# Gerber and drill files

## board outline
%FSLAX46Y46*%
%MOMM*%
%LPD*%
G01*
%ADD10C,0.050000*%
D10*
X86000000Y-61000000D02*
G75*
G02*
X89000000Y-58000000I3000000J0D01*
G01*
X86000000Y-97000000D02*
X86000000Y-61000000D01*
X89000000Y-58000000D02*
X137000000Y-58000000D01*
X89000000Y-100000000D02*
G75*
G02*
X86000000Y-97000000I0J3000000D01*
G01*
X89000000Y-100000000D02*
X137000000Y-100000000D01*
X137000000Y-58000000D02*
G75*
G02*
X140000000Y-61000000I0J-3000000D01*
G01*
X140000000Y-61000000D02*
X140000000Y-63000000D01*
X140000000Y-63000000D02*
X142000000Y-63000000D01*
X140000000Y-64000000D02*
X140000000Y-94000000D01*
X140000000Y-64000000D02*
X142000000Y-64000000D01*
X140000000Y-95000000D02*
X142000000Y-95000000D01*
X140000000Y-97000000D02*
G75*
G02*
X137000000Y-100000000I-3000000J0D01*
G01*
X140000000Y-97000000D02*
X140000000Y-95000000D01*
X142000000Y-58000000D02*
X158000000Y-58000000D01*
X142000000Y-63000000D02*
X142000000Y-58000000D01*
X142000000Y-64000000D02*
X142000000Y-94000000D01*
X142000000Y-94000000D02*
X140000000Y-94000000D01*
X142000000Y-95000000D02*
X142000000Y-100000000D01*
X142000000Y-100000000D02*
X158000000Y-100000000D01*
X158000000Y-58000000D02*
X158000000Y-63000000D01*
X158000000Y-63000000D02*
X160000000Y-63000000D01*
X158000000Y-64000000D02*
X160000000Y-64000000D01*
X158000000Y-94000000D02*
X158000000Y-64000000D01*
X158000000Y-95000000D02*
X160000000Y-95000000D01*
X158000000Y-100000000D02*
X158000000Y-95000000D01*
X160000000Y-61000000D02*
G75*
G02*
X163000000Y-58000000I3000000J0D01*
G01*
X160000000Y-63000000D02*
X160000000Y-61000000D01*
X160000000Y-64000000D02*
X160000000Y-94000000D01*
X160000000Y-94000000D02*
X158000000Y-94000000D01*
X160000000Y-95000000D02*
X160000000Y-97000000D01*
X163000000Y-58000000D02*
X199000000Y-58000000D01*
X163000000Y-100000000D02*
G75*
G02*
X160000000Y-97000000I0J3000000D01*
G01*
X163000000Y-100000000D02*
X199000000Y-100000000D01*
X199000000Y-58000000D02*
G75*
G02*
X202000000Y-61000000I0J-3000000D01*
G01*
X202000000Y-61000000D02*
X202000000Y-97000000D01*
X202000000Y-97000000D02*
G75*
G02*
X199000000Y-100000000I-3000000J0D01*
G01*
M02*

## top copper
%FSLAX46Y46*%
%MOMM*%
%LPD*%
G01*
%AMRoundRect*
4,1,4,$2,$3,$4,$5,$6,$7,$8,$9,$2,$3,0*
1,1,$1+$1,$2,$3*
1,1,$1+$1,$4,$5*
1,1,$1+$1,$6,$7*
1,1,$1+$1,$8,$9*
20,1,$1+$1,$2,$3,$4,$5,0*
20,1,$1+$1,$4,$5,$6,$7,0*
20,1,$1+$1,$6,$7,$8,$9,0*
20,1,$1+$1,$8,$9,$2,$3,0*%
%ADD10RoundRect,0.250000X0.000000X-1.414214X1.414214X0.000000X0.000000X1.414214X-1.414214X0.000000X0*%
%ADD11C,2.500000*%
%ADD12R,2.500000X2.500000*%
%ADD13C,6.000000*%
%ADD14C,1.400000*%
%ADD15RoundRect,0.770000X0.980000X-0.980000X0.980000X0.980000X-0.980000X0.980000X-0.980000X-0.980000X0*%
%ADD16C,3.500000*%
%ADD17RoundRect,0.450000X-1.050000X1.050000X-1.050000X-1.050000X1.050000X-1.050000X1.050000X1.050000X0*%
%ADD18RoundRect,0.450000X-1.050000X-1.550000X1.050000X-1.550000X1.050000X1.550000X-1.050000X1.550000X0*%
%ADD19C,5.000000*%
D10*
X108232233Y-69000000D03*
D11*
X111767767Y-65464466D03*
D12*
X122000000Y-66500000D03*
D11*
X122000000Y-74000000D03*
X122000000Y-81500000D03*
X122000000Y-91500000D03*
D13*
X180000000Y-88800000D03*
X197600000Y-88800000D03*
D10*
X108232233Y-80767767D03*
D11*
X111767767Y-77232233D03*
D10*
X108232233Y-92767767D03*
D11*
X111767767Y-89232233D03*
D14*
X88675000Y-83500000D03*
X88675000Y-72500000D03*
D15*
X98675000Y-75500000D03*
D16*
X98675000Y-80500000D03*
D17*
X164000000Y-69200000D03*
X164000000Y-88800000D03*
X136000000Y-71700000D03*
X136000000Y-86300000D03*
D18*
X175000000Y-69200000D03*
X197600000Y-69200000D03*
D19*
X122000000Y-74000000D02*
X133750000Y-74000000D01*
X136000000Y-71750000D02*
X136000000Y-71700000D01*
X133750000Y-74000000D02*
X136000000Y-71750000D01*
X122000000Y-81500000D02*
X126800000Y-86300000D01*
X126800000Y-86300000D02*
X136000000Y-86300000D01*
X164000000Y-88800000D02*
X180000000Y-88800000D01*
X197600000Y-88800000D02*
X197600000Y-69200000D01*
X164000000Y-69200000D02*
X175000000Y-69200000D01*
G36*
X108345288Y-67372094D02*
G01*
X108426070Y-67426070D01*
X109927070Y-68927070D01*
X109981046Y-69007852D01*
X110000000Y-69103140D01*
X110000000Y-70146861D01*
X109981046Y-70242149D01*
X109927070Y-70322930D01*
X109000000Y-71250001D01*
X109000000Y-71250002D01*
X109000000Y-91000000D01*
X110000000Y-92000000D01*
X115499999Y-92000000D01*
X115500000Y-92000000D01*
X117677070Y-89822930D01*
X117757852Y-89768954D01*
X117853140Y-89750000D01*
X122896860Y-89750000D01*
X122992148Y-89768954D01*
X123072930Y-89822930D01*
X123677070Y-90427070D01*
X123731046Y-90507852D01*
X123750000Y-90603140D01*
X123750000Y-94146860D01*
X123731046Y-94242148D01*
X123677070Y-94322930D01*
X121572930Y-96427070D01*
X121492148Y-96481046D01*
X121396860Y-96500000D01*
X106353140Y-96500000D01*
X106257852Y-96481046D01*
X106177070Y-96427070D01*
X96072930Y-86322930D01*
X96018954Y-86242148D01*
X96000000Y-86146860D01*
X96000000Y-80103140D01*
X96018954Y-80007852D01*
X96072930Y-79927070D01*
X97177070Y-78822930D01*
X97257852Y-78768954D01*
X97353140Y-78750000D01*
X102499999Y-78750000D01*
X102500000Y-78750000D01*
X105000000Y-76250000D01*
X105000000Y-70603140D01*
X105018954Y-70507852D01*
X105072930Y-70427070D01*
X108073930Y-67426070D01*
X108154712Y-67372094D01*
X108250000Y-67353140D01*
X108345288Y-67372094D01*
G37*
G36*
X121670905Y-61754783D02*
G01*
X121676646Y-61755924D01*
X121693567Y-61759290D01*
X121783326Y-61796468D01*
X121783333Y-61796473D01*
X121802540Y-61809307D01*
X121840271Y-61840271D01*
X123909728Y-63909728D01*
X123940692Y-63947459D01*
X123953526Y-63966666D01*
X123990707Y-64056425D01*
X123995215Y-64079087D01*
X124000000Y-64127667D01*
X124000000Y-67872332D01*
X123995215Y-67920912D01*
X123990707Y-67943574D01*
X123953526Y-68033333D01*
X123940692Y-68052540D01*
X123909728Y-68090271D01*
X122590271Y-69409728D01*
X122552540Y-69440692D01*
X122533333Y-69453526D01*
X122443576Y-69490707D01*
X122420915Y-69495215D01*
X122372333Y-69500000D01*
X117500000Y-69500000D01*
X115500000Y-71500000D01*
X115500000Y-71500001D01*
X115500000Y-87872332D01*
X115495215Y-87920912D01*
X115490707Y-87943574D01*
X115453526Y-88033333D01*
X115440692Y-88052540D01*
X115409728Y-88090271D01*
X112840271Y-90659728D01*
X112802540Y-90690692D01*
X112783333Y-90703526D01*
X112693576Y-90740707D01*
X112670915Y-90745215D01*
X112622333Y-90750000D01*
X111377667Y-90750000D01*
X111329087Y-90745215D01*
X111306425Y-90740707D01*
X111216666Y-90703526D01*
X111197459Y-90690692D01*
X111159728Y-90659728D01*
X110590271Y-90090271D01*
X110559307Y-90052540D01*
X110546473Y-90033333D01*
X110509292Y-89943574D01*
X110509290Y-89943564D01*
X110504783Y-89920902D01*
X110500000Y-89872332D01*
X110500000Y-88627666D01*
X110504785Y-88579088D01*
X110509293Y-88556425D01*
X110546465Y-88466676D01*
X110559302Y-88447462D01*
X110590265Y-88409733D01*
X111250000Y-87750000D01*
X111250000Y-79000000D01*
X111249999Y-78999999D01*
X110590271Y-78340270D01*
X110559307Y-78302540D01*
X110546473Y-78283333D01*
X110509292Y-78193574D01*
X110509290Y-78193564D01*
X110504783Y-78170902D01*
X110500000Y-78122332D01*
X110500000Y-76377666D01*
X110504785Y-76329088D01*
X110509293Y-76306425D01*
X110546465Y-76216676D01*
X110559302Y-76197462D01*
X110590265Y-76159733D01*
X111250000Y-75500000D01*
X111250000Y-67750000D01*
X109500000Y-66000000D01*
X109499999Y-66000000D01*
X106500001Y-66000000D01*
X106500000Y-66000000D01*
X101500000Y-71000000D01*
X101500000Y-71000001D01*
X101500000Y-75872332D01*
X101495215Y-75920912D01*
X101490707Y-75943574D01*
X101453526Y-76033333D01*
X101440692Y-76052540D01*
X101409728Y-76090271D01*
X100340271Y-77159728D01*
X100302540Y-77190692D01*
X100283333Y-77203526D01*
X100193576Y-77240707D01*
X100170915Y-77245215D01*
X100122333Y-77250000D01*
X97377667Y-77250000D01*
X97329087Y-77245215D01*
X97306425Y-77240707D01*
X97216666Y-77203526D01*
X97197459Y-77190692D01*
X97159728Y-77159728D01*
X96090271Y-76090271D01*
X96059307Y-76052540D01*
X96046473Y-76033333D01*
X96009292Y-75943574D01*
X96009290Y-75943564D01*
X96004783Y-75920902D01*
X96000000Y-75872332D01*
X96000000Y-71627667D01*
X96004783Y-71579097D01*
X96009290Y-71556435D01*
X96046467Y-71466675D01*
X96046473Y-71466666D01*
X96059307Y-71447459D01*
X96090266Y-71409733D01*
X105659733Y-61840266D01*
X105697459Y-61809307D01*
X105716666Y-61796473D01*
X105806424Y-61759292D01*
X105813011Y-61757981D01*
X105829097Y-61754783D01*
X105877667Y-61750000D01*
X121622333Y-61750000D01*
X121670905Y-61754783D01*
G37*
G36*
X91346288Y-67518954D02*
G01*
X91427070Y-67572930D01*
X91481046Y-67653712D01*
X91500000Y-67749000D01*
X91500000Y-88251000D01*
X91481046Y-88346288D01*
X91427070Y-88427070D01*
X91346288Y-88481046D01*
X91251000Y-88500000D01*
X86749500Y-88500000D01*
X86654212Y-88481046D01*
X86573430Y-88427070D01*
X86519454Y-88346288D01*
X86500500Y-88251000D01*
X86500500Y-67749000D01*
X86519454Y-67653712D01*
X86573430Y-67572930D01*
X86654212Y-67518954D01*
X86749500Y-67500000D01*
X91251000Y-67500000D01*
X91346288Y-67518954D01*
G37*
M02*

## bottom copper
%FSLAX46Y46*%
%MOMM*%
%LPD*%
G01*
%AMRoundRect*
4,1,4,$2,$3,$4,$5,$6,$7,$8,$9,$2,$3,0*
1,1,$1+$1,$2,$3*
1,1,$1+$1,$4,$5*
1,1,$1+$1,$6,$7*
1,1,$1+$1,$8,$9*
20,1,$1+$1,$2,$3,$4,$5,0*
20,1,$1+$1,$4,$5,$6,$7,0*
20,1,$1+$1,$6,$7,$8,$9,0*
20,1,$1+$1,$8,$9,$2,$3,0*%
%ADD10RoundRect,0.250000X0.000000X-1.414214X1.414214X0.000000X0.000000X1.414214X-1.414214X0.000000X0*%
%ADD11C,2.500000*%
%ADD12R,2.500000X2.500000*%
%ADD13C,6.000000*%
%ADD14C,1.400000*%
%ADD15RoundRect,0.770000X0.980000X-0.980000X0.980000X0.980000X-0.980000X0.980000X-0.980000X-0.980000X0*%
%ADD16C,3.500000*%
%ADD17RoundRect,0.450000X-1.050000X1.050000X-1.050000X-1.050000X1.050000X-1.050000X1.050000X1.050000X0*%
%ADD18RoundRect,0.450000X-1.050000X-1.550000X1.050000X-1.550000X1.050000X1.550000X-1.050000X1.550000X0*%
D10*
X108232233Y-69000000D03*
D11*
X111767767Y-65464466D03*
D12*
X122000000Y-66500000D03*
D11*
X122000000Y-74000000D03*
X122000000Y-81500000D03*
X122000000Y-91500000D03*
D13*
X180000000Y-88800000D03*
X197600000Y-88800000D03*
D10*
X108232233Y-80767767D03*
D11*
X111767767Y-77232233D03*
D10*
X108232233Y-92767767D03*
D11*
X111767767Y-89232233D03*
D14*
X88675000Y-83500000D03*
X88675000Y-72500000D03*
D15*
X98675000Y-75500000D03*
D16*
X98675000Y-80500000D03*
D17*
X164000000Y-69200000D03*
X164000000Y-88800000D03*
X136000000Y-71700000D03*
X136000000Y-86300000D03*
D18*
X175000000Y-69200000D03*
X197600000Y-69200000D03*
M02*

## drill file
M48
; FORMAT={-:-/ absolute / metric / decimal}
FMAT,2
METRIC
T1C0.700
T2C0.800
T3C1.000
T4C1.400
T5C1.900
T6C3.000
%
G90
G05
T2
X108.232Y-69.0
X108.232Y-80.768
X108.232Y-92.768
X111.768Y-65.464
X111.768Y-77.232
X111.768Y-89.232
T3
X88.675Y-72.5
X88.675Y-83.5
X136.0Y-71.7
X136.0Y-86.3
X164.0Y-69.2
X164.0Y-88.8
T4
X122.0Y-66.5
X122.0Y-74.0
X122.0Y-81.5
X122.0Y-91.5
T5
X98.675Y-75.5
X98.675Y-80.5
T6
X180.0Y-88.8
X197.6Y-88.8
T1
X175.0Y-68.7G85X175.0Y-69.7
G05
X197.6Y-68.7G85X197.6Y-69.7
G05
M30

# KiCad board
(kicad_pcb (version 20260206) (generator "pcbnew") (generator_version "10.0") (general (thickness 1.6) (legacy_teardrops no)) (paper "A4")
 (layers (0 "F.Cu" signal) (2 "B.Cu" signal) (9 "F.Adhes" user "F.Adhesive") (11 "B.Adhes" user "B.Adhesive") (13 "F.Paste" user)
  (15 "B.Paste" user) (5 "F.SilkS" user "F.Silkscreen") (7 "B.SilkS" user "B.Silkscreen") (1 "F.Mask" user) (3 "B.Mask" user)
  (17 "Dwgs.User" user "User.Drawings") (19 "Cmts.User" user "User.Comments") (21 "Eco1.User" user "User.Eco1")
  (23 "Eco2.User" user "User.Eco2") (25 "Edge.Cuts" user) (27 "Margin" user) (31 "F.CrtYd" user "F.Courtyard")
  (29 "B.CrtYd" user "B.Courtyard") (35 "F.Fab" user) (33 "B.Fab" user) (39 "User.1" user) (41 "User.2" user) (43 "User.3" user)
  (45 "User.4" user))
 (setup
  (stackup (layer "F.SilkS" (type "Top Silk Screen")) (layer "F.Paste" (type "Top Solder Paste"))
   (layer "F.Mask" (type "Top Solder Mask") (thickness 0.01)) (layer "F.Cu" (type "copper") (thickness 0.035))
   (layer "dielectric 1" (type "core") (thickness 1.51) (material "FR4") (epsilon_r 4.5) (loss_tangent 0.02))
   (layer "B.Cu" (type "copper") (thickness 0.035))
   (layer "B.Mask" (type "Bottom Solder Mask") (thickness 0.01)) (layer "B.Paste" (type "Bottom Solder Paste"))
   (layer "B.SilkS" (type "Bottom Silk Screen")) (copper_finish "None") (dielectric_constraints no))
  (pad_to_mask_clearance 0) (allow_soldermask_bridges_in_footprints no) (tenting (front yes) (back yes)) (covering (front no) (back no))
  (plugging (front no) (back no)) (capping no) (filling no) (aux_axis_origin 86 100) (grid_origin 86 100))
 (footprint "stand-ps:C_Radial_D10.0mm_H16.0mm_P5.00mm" (layer "F.Cu") (at 108.232233 69 45)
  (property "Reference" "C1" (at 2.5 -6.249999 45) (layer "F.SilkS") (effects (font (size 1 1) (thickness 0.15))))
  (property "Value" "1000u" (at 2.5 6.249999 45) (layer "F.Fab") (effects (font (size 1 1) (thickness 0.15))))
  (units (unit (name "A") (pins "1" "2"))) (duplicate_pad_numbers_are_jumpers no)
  (pad "1" thru_hole roundrect (at 0 0 45) (size 2.5 2.5) (drill 0.8) (layers "*.Cu" "*.Mask") (remove_unused_layers no)
   (roundrect_rratio 0.1) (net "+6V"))
  (pad "2" thru_hole circle (at 5 0 45) (size 2.5 2.5) (drill 0.8) (layers "*.Cu" "*.Mask") (remove_unused_layers no) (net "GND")))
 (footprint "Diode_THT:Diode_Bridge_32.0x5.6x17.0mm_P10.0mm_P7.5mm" (layer "F.Cu") (at 122 66.5 -90)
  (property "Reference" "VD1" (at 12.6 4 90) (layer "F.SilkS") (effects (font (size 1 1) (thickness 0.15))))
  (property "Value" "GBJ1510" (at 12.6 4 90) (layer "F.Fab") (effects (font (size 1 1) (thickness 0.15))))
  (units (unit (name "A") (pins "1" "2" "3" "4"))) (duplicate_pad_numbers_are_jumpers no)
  (pad "1" thru_hole rect (at 0 0 270) (size 2.5 2.5) (drill 1.4) (layers "*.Cu" "*.Mask") (remove_unused_layers no) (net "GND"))
  (pad "2" thru_hole circle (at 7.5 0 270) (size 2.5 2.5) (drill 1.4) (layers "*.Cu" "*.Mask") (remove_unused_layers no) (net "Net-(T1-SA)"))
  (pad "3" thru_hole circle (at 15 0 270) (size 2.5 2.5) (drill 1.4) (layers "*.Cu" "*.Mask") (remove_unused_layers no) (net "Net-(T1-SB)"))
  (pad "4" thru_hole circle (at 25 0 270) (size 2.5 2.5) (drill 1.4) (layers "*.Cu" "*.Mask") (remove_unused_layers no) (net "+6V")))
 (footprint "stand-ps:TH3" (layer "F.Cu") (at 180 88.8)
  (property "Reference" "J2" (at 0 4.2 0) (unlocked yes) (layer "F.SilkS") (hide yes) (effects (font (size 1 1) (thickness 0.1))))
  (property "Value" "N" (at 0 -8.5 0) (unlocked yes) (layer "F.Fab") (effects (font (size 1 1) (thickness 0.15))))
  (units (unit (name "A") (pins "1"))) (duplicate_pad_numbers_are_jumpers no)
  (pad "1" thru_hole circle (at 0 0) (size 6 6) (drill 3) (layers "*.Cu" "*.Mask") (remove_unused_layers no) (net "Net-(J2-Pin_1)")))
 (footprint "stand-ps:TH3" (layer "F.Cu") (at 197.6 88.8)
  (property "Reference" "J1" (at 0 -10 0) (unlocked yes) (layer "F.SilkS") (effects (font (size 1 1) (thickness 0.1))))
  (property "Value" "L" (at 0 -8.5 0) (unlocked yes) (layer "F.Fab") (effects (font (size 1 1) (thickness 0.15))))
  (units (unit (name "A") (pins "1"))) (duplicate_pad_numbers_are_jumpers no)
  (pad "1" thru_hole circle (at 0 0) (size 6 6) (drill 3) (layers "*.Cu" "*.Mask") (remove_unused_layers no) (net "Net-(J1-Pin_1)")))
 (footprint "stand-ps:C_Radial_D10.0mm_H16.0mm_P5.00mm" (layer "F.Cu") (at 108.232233 80.767767 45)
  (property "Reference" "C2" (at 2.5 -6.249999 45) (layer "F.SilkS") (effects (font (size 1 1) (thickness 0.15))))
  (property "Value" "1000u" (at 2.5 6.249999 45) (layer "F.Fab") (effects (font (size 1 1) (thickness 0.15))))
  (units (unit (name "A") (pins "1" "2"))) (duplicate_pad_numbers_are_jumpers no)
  (pad "1" thru_hole roundrect (at 0 0 45) (size 2.5 2.5) (drill 0.8) (layers "*.Cu" "*.Mask") (remove_unused_layers no)
   (roundrect_rratio 0.1) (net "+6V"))
  (pad "2" thru_hole circle (at 5 0 45) (size 2.5 2.5) (drill 0.8) (layers "*.Cu" "*.Mask") (remove_unused_layers no) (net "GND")))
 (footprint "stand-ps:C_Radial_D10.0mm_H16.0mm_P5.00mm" (layer "F.Cu") (at 108.232233 92.767767 45)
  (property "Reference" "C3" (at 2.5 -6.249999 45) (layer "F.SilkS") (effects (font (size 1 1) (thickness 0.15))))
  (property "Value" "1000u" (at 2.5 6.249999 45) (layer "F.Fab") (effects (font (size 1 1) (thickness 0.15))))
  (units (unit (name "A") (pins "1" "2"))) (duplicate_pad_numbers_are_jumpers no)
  (pad "1" thru_hole roundrect (at 0 0 45) (size 2.5 2.5) (drill 0.8) (layers "*.Cu" "*.Mask") (remove_unused_layers no)
   (roundrect_rratio 0.1) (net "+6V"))
  (pad "2" thru_hole circle (at 5 0 45) (size 2.5 2.5) (drill 0.8) (layers "*.Cu" "*.Mask") (remove_unused_layers no) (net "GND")))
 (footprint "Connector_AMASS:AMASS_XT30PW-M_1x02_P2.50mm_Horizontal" (layer "F.Cu") (at 98.675 75.5 90)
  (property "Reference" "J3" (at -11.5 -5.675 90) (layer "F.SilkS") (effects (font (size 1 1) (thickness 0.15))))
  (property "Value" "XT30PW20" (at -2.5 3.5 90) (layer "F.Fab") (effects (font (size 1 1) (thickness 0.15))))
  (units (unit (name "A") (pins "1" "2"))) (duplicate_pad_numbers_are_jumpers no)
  (pad "" thru_hole circle (at -8 -10 90) (size 1.4 1.4) (drill 1) (layers "*.Cu" "*.Mask") (remove_unused_layers no) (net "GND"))
  (pad "" thru_hole circle (at 3 -10 90) (size 1.4 1.4) (drill 1) (layers "*.Cu" "*.Mask") (remove_unused_layers no) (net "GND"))
  (pad "1" thru_hole roundrect (at 0 0 90) (size 3.5 3.5) (drill 1.9) (layers "*.Cu" "*.Mask") (remove_unused_layers no)
   (roundrect_rratio 0.22) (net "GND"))
  (pad "2" thru_hole circle (at -5 0 90) (size 3.5 3.5) (drill 1.9) (layers "*.Cu" "*.Mask") (remove_unused_layers no) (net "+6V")))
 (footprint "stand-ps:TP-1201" (layer "F.Cu") (at 164 79 -90)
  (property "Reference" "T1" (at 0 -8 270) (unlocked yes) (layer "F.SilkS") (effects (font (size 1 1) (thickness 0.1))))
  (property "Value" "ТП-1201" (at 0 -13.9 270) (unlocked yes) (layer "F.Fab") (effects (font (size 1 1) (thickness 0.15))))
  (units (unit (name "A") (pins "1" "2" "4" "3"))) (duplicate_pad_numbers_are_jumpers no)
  (pad "1" thru_hole roundrect (at -9.8 0 270) (size 3 3) (drill 1) (layers "*.Cu" "*.Mask") (remove_unused_layers no)
   (roundrect_rratio 0.15) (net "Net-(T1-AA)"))
  (pad "2" thru_hole roundrect (at 9.8 0 270) (size 3 3) (drill 1) (layers "*.Cu" "*.Mask") (remove_unused_layers no)
   (roundrect_rratio 0.15) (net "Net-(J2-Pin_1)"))
  (pad "3" thru_hole roundrect (at -7.3 28 270) (size 3 3) (drill 1) (layers "*.Cu" "*.Mask") (remove_unused_layers no)
   (roundrect_rratio 0.15) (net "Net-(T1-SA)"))
  (pad "4" thru_hole roundrect (at 7.3 28 270) (size 3 3) (drill 1) (layers "*.Cu" "*.Mask") (remove_unused_layers no)
   (roundrect_rratio 0.15) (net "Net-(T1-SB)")))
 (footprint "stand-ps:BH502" (layer "F.Cu") (at 186.3 69.2)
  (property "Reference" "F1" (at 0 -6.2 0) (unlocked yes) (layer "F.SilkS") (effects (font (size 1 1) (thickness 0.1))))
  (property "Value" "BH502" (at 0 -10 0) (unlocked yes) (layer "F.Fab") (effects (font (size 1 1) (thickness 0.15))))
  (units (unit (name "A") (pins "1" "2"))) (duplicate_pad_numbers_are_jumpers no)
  (pad "1" thru_hole roundrect (at -11.3 0) (size 3 4) (drill oval 0.7 1.7) (layers "*.Cu" "*.Mask") (remove_unused_layers no)
   (roundrect_rratio 0.15) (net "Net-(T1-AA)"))
  (pad "2" thru_hole roundrect (at 11.3 0) (size 3 4) (drill oval 0.7 1.7) (layers "*.Cu" "*.Mask") (remove_unused_layers no)
   (roundrect_rratio 0.15) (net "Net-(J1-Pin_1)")))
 (gr_arc (start 86 61) (mid 86.87868 58.87868) (end 89 58) (stroke (width 0.05) (type default)) (layer "Edge.Cuts"))
 (gr_line (start 86 97) (end 86 61) (stroke (width 0.05) (type default)) (layer "Edge.Cuts"))
 (gr_line (start 89 58) (end 137 58) (stroke (width 0.05) (type default)) (layer "Edge.Cuts"))
 (gr_arc (start 89 100) (mid 86.87868 99.12132) (end 86 97) (stroke (width 0.05) (type default)) (layer "Edge.Cuts"))
 (gr_line (start 89 100) (end 137 100) (stroke (width 0.05) (type default)) (layer "Edge.Cuts"))
 (gr_arc (start 137 58) (mid 139.12132 58.87868) (end 140 61) (stroke (width 0.05) (type default)) (layer "Edge.Cuts"))
 (gr_line (start 140 61) (end 140 63) (stroke (width 0.05) (type default)) (layer "Edge.Cuts"))
 (gr_line (start 140 63) (end 142 63) (stroke (width 0.05) (type default)) (layer "Edge.Cuts"))
 (gr_line (start 140 64) (end 140 94) (stroke (width 0.05) (type default)) (layer "Edge.Cuts"))
 (gr_line (start 140 64) (end 142 64) (stroke (width 0.05) (type default)) (layer "Edge.Cuts"))
 (gr_line (start 140 95) (end 142 95) (stroke (width 0.05) (type default)) (layer "Edge.Cuts"))
 (gr_arc (start 140 97) (mid 139.12132 99.12132) (end 137 100) (stroke (width 0.05) (type default)) (layer "Edge.Cuts"))
 (gr_line (start 140 97) (end 140 95) (stroke (width 0.05) (type default)) (layer "Edge.Cuts"))
 (gr_line (start 142 58) (end 158 58) (stroke (width 0.05) (type default)) (layer "Edge.Cuts"))
 (gr_line (start 142 63) (end 142 58) (stroke (width 0.05) (type default)) (layer "Edge.Cuts"))
 (gr_line (start 142 64) (end 142 94) (stroke (width 0.05) (type default)) (layer "Edge.Cuts"))
 (gr_line (start 142 94) (end 140 94) (stroke (width 0.05) (type default)) (layer "Edge.Cuts"))
 (gr_line (start 142 95) (end 142 100) (stroke (width 0.05) (type default)) (layer "Edge.Cuts"))
 (gr_line (start 142 100) (end 158 100) (stroke (width 0.05) (type default)) (layer "Edge.Cuts"))
 (gr_line (start 158 58) (end 158 63) (stroke (width 0.05) (type default)) (layer "Edge.Cuts"))
 (gr_line (start 158 63) (end 160 63) (stroke (width 0.05) (type default)) (layer "Edge.Cuts"))
 (gr_line (start 158 64) (end 160 64) (stroke (width 0.05) (type default)) (layer "Edge.Cuts"))
 (gr_line (start 158 94) (end 158 64) (stroke (width 0.05) (type default)) (layer "Edge.Cuts"))
 (gr_line (start 158 95) (end 160 95) (stroke (width 0.05) (type default)) (layer "Edge.Cuts"))
 (gr_line (start 158 100) (end 158 95) (stroke (width 0.05) (type default)) (layer "Edge.Cuts"))
 (gr_arc (start 160 61) (mid 160.87868 58.87868) (end 163 58) (stroke (width 0.05) (type default)) (layer "Edge.Cuts"))
 (gr_line (start 160 63) (end 160 61) (stroke (width 0.05) (type default)) (layer "Edge.Cuts"))
 (gr_line (start 160 64) (end 160 94) (stroke (width 0.05) (type default)) (layer "Edge.Cuts"))
 (gr_line (start 160 94) (end 158 94) (stroke (width 0.05) (type default)) (layer "Edge.Cuts"))
 (gr_line (start 160 95) (end 160 97) (stroke (width 0.05) (type default)) (layer "Edge.Cuts"))
 (gr_line (start 163 58) (end 199 58) (stroke (width 0.05) (type default)) (layer "Edge.Cuts"))
 (gr_arc (start 163 100) (mid 160.87868 99.12132) (end 160 97) (stroke (width 0.05) (type default)) (layer "Edge.Cuts"))
 (gr_line (start 163 100) (end 199 100) (stroke (width 0.05) (type default)) (layer "Edge.Cuts"))
 (gr_arc (start 199 58) (mid 201.12132 58.87868) (end 202 61) (stroke (width 0.05) (type default)) (layer "Edge.Cuts"))
 (gr_line (start 202 61) (end 202 97) (stroke (width 0.05) (type default)) (layer "Edge.Cuts"))
 (gr_arc (start 202 97) (mid 201.12132 99.12132) (end 199 100) (stroke (width 0.05) (type default)) (layer "Edge.Cuts"))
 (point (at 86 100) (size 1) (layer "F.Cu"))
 (segment (start 122 74) (end 133.75 74) (width 5) (layer "F.Cu") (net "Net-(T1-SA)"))
 (segment (start 136 71.75) (end 136 71.7) (width 5) (layer "F.Cu") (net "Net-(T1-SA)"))
 (segment (start 133.75 74) (end 136 71.75) (width 5) (layer "F.Cu") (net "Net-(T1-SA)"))
 (segment (start 122 81.5) (end 126.8 86.3) (width 5) (layer "F.Cu") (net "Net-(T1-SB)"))
 (segment (start 126.8 86.3) (end 136 86.3) (width 5) (layer "F.Cu") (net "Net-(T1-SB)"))
 (segment (start 164 88.8) (end 180 88.8) (width 5) (layer "F.Cu") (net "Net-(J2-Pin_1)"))
 (segment (start 197.6 88.8) (end 197.6 69.2) (width 5) (layer "F.Cu") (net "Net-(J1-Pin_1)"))
 (segment (start 164 69.2) (end 175 69.2) (width 5) (layer "F.Cu") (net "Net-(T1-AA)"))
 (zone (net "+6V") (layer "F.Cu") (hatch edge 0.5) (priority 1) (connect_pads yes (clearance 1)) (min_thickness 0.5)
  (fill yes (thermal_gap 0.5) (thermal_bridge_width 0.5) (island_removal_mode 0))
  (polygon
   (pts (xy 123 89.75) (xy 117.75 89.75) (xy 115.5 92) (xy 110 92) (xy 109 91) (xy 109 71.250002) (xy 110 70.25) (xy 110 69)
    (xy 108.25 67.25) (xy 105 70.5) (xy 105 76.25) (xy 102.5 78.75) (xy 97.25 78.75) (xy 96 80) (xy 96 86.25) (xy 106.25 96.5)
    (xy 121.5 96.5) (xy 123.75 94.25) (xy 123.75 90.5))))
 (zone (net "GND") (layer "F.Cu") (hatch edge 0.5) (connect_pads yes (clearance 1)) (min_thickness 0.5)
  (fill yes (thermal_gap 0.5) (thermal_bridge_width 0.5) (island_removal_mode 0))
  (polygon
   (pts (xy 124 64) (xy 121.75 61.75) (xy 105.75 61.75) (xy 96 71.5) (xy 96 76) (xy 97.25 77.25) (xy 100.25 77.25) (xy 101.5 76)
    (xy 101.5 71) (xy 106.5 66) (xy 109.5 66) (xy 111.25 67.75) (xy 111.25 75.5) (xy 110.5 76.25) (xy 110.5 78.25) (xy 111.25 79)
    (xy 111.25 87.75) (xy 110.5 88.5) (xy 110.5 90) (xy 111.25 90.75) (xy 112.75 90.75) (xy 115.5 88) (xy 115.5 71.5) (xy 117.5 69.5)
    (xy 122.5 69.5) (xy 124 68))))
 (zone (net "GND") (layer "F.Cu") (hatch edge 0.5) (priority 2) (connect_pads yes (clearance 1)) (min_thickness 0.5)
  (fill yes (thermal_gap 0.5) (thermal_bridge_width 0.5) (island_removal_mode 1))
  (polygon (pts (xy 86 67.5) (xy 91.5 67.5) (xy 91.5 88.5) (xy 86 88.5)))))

